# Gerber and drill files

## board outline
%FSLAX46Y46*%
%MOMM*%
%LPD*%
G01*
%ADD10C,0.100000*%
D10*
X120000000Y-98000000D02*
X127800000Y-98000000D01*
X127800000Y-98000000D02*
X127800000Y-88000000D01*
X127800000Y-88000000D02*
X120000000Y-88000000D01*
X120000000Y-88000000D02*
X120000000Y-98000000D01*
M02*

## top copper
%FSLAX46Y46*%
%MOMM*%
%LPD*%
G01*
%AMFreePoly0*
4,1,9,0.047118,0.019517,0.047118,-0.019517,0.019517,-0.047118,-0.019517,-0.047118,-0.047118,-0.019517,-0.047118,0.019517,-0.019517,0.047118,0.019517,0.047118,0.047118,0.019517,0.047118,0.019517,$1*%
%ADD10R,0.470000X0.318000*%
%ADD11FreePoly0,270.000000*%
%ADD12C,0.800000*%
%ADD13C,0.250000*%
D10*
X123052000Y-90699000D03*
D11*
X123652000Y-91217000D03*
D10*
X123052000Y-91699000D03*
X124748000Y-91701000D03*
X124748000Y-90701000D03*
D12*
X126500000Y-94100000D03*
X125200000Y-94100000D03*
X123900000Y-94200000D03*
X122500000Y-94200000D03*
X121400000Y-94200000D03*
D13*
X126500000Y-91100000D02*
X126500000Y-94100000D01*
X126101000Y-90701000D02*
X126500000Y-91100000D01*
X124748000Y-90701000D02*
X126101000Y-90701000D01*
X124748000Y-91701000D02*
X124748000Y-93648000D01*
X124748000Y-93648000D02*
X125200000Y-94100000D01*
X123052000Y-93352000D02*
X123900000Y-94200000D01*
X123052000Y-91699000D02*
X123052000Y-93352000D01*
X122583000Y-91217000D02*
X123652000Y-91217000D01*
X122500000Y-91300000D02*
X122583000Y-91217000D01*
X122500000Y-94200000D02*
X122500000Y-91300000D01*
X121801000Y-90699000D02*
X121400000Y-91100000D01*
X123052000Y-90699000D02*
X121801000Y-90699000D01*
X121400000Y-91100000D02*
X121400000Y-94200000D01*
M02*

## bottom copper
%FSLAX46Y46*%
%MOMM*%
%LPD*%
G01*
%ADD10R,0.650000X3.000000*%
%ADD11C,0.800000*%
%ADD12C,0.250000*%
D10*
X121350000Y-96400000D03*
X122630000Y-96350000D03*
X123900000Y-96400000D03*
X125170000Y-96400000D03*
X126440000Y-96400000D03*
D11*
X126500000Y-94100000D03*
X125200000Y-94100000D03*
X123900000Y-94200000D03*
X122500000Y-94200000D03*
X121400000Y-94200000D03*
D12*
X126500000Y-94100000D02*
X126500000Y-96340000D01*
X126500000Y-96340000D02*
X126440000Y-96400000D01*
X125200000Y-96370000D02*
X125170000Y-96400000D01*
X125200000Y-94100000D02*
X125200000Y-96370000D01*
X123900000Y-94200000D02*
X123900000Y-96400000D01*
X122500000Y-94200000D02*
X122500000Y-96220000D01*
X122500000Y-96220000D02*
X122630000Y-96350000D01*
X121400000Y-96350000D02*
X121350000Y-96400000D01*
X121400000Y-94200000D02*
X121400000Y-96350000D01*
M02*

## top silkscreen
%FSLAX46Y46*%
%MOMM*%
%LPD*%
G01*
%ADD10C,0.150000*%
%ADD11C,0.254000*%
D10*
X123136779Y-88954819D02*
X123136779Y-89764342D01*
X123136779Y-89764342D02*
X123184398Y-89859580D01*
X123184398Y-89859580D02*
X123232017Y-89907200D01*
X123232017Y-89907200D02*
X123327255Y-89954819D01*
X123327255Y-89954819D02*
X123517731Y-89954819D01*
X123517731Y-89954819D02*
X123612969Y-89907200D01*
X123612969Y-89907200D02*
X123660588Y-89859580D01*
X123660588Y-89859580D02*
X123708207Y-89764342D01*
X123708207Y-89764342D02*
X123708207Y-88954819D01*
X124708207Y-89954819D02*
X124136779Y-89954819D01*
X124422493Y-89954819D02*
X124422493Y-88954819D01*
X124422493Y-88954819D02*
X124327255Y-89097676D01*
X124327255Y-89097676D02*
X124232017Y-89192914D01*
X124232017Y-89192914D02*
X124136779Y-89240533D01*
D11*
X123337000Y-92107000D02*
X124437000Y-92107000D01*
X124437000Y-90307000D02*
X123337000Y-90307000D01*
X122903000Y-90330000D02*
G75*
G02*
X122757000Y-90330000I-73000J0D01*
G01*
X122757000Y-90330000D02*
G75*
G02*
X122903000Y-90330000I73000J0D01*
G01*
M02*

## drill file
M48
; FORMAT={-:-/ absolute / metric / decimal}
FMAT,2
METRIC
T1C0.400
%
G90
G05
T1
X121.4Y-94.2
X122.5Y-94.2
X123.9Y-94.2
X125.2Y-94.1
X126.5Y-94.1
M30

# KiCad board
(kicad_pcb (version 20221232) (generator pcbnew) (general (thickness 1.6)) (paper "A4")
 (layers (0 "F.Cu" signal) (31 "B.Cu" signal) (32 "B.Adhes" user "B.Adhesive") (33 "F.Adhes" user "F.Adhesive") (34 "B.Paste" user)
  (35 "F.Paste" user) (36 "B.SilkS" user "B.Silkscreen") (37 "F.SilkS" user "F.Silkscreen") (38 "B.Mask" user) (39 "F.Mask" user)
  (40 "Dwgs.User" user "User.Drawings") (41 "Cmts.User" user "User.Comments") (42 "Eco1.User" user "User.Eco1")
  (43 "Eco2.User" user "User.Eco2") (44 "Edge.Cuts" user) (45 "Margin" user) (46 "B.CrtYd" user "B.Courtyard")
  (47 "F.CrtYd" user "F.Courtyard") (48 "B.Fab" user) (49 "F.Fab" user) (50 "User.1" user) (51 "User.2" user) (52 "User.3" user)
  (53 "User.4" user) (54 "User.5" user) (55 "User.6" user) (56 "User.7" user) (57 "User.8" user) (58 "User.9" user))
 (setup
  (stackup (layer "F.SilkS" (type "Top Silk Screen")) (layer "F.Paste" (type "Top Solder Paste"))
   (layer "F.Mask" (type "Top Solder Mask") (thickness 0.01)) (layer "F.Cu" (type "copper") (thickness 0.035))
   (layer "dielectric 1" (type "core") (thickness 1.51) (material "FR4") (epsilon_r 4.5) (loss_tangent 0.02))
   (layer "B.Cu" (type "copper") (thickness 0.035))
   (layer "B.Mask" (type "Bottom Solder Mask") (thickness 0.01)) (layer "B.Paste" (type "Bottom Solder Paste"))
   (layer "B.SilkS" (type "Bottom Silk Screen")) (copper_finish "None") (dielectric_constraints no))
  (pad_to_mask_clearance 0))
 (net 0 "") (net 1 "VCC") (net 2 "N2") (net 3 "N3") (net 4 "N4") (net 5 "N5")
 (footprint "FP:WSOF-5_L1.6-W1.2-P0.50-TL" (layer "F.Cu") (at 123.9 91.2)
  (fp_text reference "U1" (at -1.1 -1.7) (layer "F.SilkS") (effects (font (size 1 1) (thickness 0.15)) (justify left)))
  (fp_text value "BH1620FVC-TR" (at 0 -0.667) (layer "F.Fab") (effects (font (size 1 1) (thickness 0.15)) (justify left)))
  (fp_line (start -0.563 0.907) (end 0.537 0.907) (stroke (width 0.254) (type solid)) (layer "F.SilkS"))
  (fp_line (start 0.537 -0.893) (end -0.563 -0.893) (stroke (width 0.254) (type solid)) (layer "F.SilkS"))
  (fp_circle (center -1.07 -0.87) (end -0.997 -0.87) (stroke (width 0.254) (type solid)) (fill none) (layer "F.SilkS"))
  (pad "1" smd rect locked (at -0.848 -0.501 90) (size 0.318 0.47) (layers "F.Cu" "F.Paste" "F.Mask") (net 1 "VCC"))
  (pad "2" smd custom locked (at -0.248 0.017 270) (size 0.102 0.102) (layers "F.Cu" "F.Paste" "F.Mask") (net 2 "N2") (zone_connect 0)
   (thermal_bridge_angle 45) (options (clearance outline) (anchor circle)) (primitives))
  (pad "3" smd rect locked (at -0.848 0.499 90) (size 0.318 0.47) (layers "F.Cu" "F.Paste" "F.Mask") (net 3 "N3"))
  (pad "4" smd rect locked (at 0.848 0.501 90) (size 0.318 0.47) (layers "F.Cu" "F.Paste" "F.Mask") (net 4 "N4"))
  (pad "5" smd rect locked (at 0.848 -0.499 90) (size 0.318 0.47) (layers "F.Cu" "F.Paste" "F.Mask") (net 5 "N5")))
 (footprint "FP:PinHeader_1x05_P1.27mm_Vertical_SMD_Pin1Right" (layer "B.Cu") (at 123.9 96.8 -90)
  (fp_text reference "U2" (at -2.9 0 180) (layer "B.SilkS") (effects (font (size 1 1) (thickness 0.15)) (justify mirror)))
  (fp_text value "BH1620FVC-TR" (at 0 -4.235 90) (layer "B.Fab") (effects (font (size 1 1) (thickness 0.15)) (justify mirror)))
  (pad "1" smd rect (at -0.4 2.55 270) (size 3 0.65) (layers "B.Cu" "B.Paste" "B.Mask") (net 1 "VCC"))
  (pad "2" smd rect (at -0.45 1.27 270) (size 3 0.65) (layers "B.Cu" "B.Paste" "B.Mask") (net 2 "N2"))
  (pad "3" smd rect (at -0.4 0 270) (size 3 0.65) (layers "B.Cu" "B.Paste" "B.Mask") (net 3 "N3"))
  (pad "4" smd rect (at -0.4 -1.27 270) (size 3 0.65) (layers "B.Cu" "B.Paste" "B.Mask") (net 4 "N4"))
  (pad "5" smd rect (at -0.4 -2.54 270) (size 3 0.65) (layers "B.Cu" "B.Paste" "B.Mask") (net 5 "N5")))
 (gr_line (start 120 98) (end 127.8 98) (stroke (width 0.1) (type default)) (layer "Edge.Cuts"))
 (gr_line (start 127.8 98) (end 127.8 88) (stroke (width 0.1) (type default)) (layer "Edge.Cuts"))
 (gr_line (start 127.8 88) (end 120 88) (stroke (width 0.1) (type default)) (layer "Edge.Cuts"))
 (gr_line (start 120 88) (end 120 98) (stroke (width 0.1) (type default)) (layer "Edge.Cuts"))
 (segment (start 126.5 91.1) (end 126.5 94.1) (width 0.25) (layer "F.Cu") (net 5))
 (segment (start 126.101 90.701) (end 126.5 91.1) (width 0.25) (layer "F.Cu") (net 5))
 (segment (start 124.748 90.701) (end 126.101 90.701) (width 0.25) (layer "F.Cu") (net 5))
 (via (at 126.5 94.1) (size 0.8) (drill 0.4) (layers "F.Cu" "B.Cu") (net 5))
 (segment (start 126.5 94.1) (end 126.5 96.34) (width 0.25) (layer "B.Cu") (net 5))
 (segment (start 126.5 96.34) (end 126.44 96.4) (width 0.25) (layer "B.Cu") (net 5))
 (segment (start 124.748 91.701) (end 124.748 93.648) (width 0.25) (layer "F.Cu") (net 4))
 (segment (start 124.748 93.648) (end 125.2 94.1) (width 0.25) (layer "F.Cu") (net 4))
 (via (at 125.2 94.1) (size 0.8) (drill 0.4) (layers "F.Cu" "B.Cu") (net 4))
 (segment (start 125.2 96.37) (end 125.17 96.4) (width 0.25) (layer "B.Cu") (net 4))
 (segment (start 125.2 94.1) (end 125.2 96.37) (width 0.25) (layer "B.Cu") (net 4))
 (segment (start 123.052 93.352) (end 123.9 94.2) (width 0.25) (layer "F.Cu") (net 3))
 (segment (start 123.052 91.699) (end 123.052 93.352) (width 0.25) (layer "F.Cu") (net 3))
 (via (at 123.9 94.2) (size 0.8) (drill 0.4) (layers "F.Cu" "B.Cu") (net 3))
 (segment (start 123.9 94.2) (end 123.9 96.4) (width 0.25) (layer "B.Cu") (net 3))
 (segment (start 122.583 91.217) (end 123.652 91.217) (width 0.25) (layer "F.Cu") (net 2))
 (segment (start 122.5 91.3) (end 122.583 91.217) (width 0.25) (layer "F.Cu") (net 2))
 (segment (start 122.5 94.2) (end 122.5 91.3) (width 0.25) (layer "F.Cu") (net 2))
 (via (at 122.5 94.2) (size 0.8) (drill 0.4) (layers "F.Cu" "B.Cu") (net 2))
 (segment (start 122.5 94.2) (end 122.5 96.22) (width 0.25) (layer "B.Cu") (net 2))
 (segment (start 122.5 96.22) (end 122.63 96.35) (width 0.25) (layer "B.Cu") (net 2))
 (segment (start 121.801 90.699) (end 121.4 91.1) (width 0.25) (layer "F.Cu") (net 1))
 (segment (start 123.052 90.699) (end 121.801 90.699) (width 0.25) (layer "F.Cu") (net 1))
 (segment (start 121.4 91.1) (end 121.4 94.2) (width 0.25) (layer "F.Cu") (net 1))
 (via (at 121.4 94.2) (size 0.8) (drill 0.4) (layers "F.Cu" "B.Cu") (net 1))
 (segment (start 121.4 96.35) (end 121.35 96.4) (width 0.25) (layer "B.Cu") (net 1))
 (segment (start 121.4 94.2) (end 121.4 96.35) (width 0.25) (layer "B.Cu") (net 1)))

